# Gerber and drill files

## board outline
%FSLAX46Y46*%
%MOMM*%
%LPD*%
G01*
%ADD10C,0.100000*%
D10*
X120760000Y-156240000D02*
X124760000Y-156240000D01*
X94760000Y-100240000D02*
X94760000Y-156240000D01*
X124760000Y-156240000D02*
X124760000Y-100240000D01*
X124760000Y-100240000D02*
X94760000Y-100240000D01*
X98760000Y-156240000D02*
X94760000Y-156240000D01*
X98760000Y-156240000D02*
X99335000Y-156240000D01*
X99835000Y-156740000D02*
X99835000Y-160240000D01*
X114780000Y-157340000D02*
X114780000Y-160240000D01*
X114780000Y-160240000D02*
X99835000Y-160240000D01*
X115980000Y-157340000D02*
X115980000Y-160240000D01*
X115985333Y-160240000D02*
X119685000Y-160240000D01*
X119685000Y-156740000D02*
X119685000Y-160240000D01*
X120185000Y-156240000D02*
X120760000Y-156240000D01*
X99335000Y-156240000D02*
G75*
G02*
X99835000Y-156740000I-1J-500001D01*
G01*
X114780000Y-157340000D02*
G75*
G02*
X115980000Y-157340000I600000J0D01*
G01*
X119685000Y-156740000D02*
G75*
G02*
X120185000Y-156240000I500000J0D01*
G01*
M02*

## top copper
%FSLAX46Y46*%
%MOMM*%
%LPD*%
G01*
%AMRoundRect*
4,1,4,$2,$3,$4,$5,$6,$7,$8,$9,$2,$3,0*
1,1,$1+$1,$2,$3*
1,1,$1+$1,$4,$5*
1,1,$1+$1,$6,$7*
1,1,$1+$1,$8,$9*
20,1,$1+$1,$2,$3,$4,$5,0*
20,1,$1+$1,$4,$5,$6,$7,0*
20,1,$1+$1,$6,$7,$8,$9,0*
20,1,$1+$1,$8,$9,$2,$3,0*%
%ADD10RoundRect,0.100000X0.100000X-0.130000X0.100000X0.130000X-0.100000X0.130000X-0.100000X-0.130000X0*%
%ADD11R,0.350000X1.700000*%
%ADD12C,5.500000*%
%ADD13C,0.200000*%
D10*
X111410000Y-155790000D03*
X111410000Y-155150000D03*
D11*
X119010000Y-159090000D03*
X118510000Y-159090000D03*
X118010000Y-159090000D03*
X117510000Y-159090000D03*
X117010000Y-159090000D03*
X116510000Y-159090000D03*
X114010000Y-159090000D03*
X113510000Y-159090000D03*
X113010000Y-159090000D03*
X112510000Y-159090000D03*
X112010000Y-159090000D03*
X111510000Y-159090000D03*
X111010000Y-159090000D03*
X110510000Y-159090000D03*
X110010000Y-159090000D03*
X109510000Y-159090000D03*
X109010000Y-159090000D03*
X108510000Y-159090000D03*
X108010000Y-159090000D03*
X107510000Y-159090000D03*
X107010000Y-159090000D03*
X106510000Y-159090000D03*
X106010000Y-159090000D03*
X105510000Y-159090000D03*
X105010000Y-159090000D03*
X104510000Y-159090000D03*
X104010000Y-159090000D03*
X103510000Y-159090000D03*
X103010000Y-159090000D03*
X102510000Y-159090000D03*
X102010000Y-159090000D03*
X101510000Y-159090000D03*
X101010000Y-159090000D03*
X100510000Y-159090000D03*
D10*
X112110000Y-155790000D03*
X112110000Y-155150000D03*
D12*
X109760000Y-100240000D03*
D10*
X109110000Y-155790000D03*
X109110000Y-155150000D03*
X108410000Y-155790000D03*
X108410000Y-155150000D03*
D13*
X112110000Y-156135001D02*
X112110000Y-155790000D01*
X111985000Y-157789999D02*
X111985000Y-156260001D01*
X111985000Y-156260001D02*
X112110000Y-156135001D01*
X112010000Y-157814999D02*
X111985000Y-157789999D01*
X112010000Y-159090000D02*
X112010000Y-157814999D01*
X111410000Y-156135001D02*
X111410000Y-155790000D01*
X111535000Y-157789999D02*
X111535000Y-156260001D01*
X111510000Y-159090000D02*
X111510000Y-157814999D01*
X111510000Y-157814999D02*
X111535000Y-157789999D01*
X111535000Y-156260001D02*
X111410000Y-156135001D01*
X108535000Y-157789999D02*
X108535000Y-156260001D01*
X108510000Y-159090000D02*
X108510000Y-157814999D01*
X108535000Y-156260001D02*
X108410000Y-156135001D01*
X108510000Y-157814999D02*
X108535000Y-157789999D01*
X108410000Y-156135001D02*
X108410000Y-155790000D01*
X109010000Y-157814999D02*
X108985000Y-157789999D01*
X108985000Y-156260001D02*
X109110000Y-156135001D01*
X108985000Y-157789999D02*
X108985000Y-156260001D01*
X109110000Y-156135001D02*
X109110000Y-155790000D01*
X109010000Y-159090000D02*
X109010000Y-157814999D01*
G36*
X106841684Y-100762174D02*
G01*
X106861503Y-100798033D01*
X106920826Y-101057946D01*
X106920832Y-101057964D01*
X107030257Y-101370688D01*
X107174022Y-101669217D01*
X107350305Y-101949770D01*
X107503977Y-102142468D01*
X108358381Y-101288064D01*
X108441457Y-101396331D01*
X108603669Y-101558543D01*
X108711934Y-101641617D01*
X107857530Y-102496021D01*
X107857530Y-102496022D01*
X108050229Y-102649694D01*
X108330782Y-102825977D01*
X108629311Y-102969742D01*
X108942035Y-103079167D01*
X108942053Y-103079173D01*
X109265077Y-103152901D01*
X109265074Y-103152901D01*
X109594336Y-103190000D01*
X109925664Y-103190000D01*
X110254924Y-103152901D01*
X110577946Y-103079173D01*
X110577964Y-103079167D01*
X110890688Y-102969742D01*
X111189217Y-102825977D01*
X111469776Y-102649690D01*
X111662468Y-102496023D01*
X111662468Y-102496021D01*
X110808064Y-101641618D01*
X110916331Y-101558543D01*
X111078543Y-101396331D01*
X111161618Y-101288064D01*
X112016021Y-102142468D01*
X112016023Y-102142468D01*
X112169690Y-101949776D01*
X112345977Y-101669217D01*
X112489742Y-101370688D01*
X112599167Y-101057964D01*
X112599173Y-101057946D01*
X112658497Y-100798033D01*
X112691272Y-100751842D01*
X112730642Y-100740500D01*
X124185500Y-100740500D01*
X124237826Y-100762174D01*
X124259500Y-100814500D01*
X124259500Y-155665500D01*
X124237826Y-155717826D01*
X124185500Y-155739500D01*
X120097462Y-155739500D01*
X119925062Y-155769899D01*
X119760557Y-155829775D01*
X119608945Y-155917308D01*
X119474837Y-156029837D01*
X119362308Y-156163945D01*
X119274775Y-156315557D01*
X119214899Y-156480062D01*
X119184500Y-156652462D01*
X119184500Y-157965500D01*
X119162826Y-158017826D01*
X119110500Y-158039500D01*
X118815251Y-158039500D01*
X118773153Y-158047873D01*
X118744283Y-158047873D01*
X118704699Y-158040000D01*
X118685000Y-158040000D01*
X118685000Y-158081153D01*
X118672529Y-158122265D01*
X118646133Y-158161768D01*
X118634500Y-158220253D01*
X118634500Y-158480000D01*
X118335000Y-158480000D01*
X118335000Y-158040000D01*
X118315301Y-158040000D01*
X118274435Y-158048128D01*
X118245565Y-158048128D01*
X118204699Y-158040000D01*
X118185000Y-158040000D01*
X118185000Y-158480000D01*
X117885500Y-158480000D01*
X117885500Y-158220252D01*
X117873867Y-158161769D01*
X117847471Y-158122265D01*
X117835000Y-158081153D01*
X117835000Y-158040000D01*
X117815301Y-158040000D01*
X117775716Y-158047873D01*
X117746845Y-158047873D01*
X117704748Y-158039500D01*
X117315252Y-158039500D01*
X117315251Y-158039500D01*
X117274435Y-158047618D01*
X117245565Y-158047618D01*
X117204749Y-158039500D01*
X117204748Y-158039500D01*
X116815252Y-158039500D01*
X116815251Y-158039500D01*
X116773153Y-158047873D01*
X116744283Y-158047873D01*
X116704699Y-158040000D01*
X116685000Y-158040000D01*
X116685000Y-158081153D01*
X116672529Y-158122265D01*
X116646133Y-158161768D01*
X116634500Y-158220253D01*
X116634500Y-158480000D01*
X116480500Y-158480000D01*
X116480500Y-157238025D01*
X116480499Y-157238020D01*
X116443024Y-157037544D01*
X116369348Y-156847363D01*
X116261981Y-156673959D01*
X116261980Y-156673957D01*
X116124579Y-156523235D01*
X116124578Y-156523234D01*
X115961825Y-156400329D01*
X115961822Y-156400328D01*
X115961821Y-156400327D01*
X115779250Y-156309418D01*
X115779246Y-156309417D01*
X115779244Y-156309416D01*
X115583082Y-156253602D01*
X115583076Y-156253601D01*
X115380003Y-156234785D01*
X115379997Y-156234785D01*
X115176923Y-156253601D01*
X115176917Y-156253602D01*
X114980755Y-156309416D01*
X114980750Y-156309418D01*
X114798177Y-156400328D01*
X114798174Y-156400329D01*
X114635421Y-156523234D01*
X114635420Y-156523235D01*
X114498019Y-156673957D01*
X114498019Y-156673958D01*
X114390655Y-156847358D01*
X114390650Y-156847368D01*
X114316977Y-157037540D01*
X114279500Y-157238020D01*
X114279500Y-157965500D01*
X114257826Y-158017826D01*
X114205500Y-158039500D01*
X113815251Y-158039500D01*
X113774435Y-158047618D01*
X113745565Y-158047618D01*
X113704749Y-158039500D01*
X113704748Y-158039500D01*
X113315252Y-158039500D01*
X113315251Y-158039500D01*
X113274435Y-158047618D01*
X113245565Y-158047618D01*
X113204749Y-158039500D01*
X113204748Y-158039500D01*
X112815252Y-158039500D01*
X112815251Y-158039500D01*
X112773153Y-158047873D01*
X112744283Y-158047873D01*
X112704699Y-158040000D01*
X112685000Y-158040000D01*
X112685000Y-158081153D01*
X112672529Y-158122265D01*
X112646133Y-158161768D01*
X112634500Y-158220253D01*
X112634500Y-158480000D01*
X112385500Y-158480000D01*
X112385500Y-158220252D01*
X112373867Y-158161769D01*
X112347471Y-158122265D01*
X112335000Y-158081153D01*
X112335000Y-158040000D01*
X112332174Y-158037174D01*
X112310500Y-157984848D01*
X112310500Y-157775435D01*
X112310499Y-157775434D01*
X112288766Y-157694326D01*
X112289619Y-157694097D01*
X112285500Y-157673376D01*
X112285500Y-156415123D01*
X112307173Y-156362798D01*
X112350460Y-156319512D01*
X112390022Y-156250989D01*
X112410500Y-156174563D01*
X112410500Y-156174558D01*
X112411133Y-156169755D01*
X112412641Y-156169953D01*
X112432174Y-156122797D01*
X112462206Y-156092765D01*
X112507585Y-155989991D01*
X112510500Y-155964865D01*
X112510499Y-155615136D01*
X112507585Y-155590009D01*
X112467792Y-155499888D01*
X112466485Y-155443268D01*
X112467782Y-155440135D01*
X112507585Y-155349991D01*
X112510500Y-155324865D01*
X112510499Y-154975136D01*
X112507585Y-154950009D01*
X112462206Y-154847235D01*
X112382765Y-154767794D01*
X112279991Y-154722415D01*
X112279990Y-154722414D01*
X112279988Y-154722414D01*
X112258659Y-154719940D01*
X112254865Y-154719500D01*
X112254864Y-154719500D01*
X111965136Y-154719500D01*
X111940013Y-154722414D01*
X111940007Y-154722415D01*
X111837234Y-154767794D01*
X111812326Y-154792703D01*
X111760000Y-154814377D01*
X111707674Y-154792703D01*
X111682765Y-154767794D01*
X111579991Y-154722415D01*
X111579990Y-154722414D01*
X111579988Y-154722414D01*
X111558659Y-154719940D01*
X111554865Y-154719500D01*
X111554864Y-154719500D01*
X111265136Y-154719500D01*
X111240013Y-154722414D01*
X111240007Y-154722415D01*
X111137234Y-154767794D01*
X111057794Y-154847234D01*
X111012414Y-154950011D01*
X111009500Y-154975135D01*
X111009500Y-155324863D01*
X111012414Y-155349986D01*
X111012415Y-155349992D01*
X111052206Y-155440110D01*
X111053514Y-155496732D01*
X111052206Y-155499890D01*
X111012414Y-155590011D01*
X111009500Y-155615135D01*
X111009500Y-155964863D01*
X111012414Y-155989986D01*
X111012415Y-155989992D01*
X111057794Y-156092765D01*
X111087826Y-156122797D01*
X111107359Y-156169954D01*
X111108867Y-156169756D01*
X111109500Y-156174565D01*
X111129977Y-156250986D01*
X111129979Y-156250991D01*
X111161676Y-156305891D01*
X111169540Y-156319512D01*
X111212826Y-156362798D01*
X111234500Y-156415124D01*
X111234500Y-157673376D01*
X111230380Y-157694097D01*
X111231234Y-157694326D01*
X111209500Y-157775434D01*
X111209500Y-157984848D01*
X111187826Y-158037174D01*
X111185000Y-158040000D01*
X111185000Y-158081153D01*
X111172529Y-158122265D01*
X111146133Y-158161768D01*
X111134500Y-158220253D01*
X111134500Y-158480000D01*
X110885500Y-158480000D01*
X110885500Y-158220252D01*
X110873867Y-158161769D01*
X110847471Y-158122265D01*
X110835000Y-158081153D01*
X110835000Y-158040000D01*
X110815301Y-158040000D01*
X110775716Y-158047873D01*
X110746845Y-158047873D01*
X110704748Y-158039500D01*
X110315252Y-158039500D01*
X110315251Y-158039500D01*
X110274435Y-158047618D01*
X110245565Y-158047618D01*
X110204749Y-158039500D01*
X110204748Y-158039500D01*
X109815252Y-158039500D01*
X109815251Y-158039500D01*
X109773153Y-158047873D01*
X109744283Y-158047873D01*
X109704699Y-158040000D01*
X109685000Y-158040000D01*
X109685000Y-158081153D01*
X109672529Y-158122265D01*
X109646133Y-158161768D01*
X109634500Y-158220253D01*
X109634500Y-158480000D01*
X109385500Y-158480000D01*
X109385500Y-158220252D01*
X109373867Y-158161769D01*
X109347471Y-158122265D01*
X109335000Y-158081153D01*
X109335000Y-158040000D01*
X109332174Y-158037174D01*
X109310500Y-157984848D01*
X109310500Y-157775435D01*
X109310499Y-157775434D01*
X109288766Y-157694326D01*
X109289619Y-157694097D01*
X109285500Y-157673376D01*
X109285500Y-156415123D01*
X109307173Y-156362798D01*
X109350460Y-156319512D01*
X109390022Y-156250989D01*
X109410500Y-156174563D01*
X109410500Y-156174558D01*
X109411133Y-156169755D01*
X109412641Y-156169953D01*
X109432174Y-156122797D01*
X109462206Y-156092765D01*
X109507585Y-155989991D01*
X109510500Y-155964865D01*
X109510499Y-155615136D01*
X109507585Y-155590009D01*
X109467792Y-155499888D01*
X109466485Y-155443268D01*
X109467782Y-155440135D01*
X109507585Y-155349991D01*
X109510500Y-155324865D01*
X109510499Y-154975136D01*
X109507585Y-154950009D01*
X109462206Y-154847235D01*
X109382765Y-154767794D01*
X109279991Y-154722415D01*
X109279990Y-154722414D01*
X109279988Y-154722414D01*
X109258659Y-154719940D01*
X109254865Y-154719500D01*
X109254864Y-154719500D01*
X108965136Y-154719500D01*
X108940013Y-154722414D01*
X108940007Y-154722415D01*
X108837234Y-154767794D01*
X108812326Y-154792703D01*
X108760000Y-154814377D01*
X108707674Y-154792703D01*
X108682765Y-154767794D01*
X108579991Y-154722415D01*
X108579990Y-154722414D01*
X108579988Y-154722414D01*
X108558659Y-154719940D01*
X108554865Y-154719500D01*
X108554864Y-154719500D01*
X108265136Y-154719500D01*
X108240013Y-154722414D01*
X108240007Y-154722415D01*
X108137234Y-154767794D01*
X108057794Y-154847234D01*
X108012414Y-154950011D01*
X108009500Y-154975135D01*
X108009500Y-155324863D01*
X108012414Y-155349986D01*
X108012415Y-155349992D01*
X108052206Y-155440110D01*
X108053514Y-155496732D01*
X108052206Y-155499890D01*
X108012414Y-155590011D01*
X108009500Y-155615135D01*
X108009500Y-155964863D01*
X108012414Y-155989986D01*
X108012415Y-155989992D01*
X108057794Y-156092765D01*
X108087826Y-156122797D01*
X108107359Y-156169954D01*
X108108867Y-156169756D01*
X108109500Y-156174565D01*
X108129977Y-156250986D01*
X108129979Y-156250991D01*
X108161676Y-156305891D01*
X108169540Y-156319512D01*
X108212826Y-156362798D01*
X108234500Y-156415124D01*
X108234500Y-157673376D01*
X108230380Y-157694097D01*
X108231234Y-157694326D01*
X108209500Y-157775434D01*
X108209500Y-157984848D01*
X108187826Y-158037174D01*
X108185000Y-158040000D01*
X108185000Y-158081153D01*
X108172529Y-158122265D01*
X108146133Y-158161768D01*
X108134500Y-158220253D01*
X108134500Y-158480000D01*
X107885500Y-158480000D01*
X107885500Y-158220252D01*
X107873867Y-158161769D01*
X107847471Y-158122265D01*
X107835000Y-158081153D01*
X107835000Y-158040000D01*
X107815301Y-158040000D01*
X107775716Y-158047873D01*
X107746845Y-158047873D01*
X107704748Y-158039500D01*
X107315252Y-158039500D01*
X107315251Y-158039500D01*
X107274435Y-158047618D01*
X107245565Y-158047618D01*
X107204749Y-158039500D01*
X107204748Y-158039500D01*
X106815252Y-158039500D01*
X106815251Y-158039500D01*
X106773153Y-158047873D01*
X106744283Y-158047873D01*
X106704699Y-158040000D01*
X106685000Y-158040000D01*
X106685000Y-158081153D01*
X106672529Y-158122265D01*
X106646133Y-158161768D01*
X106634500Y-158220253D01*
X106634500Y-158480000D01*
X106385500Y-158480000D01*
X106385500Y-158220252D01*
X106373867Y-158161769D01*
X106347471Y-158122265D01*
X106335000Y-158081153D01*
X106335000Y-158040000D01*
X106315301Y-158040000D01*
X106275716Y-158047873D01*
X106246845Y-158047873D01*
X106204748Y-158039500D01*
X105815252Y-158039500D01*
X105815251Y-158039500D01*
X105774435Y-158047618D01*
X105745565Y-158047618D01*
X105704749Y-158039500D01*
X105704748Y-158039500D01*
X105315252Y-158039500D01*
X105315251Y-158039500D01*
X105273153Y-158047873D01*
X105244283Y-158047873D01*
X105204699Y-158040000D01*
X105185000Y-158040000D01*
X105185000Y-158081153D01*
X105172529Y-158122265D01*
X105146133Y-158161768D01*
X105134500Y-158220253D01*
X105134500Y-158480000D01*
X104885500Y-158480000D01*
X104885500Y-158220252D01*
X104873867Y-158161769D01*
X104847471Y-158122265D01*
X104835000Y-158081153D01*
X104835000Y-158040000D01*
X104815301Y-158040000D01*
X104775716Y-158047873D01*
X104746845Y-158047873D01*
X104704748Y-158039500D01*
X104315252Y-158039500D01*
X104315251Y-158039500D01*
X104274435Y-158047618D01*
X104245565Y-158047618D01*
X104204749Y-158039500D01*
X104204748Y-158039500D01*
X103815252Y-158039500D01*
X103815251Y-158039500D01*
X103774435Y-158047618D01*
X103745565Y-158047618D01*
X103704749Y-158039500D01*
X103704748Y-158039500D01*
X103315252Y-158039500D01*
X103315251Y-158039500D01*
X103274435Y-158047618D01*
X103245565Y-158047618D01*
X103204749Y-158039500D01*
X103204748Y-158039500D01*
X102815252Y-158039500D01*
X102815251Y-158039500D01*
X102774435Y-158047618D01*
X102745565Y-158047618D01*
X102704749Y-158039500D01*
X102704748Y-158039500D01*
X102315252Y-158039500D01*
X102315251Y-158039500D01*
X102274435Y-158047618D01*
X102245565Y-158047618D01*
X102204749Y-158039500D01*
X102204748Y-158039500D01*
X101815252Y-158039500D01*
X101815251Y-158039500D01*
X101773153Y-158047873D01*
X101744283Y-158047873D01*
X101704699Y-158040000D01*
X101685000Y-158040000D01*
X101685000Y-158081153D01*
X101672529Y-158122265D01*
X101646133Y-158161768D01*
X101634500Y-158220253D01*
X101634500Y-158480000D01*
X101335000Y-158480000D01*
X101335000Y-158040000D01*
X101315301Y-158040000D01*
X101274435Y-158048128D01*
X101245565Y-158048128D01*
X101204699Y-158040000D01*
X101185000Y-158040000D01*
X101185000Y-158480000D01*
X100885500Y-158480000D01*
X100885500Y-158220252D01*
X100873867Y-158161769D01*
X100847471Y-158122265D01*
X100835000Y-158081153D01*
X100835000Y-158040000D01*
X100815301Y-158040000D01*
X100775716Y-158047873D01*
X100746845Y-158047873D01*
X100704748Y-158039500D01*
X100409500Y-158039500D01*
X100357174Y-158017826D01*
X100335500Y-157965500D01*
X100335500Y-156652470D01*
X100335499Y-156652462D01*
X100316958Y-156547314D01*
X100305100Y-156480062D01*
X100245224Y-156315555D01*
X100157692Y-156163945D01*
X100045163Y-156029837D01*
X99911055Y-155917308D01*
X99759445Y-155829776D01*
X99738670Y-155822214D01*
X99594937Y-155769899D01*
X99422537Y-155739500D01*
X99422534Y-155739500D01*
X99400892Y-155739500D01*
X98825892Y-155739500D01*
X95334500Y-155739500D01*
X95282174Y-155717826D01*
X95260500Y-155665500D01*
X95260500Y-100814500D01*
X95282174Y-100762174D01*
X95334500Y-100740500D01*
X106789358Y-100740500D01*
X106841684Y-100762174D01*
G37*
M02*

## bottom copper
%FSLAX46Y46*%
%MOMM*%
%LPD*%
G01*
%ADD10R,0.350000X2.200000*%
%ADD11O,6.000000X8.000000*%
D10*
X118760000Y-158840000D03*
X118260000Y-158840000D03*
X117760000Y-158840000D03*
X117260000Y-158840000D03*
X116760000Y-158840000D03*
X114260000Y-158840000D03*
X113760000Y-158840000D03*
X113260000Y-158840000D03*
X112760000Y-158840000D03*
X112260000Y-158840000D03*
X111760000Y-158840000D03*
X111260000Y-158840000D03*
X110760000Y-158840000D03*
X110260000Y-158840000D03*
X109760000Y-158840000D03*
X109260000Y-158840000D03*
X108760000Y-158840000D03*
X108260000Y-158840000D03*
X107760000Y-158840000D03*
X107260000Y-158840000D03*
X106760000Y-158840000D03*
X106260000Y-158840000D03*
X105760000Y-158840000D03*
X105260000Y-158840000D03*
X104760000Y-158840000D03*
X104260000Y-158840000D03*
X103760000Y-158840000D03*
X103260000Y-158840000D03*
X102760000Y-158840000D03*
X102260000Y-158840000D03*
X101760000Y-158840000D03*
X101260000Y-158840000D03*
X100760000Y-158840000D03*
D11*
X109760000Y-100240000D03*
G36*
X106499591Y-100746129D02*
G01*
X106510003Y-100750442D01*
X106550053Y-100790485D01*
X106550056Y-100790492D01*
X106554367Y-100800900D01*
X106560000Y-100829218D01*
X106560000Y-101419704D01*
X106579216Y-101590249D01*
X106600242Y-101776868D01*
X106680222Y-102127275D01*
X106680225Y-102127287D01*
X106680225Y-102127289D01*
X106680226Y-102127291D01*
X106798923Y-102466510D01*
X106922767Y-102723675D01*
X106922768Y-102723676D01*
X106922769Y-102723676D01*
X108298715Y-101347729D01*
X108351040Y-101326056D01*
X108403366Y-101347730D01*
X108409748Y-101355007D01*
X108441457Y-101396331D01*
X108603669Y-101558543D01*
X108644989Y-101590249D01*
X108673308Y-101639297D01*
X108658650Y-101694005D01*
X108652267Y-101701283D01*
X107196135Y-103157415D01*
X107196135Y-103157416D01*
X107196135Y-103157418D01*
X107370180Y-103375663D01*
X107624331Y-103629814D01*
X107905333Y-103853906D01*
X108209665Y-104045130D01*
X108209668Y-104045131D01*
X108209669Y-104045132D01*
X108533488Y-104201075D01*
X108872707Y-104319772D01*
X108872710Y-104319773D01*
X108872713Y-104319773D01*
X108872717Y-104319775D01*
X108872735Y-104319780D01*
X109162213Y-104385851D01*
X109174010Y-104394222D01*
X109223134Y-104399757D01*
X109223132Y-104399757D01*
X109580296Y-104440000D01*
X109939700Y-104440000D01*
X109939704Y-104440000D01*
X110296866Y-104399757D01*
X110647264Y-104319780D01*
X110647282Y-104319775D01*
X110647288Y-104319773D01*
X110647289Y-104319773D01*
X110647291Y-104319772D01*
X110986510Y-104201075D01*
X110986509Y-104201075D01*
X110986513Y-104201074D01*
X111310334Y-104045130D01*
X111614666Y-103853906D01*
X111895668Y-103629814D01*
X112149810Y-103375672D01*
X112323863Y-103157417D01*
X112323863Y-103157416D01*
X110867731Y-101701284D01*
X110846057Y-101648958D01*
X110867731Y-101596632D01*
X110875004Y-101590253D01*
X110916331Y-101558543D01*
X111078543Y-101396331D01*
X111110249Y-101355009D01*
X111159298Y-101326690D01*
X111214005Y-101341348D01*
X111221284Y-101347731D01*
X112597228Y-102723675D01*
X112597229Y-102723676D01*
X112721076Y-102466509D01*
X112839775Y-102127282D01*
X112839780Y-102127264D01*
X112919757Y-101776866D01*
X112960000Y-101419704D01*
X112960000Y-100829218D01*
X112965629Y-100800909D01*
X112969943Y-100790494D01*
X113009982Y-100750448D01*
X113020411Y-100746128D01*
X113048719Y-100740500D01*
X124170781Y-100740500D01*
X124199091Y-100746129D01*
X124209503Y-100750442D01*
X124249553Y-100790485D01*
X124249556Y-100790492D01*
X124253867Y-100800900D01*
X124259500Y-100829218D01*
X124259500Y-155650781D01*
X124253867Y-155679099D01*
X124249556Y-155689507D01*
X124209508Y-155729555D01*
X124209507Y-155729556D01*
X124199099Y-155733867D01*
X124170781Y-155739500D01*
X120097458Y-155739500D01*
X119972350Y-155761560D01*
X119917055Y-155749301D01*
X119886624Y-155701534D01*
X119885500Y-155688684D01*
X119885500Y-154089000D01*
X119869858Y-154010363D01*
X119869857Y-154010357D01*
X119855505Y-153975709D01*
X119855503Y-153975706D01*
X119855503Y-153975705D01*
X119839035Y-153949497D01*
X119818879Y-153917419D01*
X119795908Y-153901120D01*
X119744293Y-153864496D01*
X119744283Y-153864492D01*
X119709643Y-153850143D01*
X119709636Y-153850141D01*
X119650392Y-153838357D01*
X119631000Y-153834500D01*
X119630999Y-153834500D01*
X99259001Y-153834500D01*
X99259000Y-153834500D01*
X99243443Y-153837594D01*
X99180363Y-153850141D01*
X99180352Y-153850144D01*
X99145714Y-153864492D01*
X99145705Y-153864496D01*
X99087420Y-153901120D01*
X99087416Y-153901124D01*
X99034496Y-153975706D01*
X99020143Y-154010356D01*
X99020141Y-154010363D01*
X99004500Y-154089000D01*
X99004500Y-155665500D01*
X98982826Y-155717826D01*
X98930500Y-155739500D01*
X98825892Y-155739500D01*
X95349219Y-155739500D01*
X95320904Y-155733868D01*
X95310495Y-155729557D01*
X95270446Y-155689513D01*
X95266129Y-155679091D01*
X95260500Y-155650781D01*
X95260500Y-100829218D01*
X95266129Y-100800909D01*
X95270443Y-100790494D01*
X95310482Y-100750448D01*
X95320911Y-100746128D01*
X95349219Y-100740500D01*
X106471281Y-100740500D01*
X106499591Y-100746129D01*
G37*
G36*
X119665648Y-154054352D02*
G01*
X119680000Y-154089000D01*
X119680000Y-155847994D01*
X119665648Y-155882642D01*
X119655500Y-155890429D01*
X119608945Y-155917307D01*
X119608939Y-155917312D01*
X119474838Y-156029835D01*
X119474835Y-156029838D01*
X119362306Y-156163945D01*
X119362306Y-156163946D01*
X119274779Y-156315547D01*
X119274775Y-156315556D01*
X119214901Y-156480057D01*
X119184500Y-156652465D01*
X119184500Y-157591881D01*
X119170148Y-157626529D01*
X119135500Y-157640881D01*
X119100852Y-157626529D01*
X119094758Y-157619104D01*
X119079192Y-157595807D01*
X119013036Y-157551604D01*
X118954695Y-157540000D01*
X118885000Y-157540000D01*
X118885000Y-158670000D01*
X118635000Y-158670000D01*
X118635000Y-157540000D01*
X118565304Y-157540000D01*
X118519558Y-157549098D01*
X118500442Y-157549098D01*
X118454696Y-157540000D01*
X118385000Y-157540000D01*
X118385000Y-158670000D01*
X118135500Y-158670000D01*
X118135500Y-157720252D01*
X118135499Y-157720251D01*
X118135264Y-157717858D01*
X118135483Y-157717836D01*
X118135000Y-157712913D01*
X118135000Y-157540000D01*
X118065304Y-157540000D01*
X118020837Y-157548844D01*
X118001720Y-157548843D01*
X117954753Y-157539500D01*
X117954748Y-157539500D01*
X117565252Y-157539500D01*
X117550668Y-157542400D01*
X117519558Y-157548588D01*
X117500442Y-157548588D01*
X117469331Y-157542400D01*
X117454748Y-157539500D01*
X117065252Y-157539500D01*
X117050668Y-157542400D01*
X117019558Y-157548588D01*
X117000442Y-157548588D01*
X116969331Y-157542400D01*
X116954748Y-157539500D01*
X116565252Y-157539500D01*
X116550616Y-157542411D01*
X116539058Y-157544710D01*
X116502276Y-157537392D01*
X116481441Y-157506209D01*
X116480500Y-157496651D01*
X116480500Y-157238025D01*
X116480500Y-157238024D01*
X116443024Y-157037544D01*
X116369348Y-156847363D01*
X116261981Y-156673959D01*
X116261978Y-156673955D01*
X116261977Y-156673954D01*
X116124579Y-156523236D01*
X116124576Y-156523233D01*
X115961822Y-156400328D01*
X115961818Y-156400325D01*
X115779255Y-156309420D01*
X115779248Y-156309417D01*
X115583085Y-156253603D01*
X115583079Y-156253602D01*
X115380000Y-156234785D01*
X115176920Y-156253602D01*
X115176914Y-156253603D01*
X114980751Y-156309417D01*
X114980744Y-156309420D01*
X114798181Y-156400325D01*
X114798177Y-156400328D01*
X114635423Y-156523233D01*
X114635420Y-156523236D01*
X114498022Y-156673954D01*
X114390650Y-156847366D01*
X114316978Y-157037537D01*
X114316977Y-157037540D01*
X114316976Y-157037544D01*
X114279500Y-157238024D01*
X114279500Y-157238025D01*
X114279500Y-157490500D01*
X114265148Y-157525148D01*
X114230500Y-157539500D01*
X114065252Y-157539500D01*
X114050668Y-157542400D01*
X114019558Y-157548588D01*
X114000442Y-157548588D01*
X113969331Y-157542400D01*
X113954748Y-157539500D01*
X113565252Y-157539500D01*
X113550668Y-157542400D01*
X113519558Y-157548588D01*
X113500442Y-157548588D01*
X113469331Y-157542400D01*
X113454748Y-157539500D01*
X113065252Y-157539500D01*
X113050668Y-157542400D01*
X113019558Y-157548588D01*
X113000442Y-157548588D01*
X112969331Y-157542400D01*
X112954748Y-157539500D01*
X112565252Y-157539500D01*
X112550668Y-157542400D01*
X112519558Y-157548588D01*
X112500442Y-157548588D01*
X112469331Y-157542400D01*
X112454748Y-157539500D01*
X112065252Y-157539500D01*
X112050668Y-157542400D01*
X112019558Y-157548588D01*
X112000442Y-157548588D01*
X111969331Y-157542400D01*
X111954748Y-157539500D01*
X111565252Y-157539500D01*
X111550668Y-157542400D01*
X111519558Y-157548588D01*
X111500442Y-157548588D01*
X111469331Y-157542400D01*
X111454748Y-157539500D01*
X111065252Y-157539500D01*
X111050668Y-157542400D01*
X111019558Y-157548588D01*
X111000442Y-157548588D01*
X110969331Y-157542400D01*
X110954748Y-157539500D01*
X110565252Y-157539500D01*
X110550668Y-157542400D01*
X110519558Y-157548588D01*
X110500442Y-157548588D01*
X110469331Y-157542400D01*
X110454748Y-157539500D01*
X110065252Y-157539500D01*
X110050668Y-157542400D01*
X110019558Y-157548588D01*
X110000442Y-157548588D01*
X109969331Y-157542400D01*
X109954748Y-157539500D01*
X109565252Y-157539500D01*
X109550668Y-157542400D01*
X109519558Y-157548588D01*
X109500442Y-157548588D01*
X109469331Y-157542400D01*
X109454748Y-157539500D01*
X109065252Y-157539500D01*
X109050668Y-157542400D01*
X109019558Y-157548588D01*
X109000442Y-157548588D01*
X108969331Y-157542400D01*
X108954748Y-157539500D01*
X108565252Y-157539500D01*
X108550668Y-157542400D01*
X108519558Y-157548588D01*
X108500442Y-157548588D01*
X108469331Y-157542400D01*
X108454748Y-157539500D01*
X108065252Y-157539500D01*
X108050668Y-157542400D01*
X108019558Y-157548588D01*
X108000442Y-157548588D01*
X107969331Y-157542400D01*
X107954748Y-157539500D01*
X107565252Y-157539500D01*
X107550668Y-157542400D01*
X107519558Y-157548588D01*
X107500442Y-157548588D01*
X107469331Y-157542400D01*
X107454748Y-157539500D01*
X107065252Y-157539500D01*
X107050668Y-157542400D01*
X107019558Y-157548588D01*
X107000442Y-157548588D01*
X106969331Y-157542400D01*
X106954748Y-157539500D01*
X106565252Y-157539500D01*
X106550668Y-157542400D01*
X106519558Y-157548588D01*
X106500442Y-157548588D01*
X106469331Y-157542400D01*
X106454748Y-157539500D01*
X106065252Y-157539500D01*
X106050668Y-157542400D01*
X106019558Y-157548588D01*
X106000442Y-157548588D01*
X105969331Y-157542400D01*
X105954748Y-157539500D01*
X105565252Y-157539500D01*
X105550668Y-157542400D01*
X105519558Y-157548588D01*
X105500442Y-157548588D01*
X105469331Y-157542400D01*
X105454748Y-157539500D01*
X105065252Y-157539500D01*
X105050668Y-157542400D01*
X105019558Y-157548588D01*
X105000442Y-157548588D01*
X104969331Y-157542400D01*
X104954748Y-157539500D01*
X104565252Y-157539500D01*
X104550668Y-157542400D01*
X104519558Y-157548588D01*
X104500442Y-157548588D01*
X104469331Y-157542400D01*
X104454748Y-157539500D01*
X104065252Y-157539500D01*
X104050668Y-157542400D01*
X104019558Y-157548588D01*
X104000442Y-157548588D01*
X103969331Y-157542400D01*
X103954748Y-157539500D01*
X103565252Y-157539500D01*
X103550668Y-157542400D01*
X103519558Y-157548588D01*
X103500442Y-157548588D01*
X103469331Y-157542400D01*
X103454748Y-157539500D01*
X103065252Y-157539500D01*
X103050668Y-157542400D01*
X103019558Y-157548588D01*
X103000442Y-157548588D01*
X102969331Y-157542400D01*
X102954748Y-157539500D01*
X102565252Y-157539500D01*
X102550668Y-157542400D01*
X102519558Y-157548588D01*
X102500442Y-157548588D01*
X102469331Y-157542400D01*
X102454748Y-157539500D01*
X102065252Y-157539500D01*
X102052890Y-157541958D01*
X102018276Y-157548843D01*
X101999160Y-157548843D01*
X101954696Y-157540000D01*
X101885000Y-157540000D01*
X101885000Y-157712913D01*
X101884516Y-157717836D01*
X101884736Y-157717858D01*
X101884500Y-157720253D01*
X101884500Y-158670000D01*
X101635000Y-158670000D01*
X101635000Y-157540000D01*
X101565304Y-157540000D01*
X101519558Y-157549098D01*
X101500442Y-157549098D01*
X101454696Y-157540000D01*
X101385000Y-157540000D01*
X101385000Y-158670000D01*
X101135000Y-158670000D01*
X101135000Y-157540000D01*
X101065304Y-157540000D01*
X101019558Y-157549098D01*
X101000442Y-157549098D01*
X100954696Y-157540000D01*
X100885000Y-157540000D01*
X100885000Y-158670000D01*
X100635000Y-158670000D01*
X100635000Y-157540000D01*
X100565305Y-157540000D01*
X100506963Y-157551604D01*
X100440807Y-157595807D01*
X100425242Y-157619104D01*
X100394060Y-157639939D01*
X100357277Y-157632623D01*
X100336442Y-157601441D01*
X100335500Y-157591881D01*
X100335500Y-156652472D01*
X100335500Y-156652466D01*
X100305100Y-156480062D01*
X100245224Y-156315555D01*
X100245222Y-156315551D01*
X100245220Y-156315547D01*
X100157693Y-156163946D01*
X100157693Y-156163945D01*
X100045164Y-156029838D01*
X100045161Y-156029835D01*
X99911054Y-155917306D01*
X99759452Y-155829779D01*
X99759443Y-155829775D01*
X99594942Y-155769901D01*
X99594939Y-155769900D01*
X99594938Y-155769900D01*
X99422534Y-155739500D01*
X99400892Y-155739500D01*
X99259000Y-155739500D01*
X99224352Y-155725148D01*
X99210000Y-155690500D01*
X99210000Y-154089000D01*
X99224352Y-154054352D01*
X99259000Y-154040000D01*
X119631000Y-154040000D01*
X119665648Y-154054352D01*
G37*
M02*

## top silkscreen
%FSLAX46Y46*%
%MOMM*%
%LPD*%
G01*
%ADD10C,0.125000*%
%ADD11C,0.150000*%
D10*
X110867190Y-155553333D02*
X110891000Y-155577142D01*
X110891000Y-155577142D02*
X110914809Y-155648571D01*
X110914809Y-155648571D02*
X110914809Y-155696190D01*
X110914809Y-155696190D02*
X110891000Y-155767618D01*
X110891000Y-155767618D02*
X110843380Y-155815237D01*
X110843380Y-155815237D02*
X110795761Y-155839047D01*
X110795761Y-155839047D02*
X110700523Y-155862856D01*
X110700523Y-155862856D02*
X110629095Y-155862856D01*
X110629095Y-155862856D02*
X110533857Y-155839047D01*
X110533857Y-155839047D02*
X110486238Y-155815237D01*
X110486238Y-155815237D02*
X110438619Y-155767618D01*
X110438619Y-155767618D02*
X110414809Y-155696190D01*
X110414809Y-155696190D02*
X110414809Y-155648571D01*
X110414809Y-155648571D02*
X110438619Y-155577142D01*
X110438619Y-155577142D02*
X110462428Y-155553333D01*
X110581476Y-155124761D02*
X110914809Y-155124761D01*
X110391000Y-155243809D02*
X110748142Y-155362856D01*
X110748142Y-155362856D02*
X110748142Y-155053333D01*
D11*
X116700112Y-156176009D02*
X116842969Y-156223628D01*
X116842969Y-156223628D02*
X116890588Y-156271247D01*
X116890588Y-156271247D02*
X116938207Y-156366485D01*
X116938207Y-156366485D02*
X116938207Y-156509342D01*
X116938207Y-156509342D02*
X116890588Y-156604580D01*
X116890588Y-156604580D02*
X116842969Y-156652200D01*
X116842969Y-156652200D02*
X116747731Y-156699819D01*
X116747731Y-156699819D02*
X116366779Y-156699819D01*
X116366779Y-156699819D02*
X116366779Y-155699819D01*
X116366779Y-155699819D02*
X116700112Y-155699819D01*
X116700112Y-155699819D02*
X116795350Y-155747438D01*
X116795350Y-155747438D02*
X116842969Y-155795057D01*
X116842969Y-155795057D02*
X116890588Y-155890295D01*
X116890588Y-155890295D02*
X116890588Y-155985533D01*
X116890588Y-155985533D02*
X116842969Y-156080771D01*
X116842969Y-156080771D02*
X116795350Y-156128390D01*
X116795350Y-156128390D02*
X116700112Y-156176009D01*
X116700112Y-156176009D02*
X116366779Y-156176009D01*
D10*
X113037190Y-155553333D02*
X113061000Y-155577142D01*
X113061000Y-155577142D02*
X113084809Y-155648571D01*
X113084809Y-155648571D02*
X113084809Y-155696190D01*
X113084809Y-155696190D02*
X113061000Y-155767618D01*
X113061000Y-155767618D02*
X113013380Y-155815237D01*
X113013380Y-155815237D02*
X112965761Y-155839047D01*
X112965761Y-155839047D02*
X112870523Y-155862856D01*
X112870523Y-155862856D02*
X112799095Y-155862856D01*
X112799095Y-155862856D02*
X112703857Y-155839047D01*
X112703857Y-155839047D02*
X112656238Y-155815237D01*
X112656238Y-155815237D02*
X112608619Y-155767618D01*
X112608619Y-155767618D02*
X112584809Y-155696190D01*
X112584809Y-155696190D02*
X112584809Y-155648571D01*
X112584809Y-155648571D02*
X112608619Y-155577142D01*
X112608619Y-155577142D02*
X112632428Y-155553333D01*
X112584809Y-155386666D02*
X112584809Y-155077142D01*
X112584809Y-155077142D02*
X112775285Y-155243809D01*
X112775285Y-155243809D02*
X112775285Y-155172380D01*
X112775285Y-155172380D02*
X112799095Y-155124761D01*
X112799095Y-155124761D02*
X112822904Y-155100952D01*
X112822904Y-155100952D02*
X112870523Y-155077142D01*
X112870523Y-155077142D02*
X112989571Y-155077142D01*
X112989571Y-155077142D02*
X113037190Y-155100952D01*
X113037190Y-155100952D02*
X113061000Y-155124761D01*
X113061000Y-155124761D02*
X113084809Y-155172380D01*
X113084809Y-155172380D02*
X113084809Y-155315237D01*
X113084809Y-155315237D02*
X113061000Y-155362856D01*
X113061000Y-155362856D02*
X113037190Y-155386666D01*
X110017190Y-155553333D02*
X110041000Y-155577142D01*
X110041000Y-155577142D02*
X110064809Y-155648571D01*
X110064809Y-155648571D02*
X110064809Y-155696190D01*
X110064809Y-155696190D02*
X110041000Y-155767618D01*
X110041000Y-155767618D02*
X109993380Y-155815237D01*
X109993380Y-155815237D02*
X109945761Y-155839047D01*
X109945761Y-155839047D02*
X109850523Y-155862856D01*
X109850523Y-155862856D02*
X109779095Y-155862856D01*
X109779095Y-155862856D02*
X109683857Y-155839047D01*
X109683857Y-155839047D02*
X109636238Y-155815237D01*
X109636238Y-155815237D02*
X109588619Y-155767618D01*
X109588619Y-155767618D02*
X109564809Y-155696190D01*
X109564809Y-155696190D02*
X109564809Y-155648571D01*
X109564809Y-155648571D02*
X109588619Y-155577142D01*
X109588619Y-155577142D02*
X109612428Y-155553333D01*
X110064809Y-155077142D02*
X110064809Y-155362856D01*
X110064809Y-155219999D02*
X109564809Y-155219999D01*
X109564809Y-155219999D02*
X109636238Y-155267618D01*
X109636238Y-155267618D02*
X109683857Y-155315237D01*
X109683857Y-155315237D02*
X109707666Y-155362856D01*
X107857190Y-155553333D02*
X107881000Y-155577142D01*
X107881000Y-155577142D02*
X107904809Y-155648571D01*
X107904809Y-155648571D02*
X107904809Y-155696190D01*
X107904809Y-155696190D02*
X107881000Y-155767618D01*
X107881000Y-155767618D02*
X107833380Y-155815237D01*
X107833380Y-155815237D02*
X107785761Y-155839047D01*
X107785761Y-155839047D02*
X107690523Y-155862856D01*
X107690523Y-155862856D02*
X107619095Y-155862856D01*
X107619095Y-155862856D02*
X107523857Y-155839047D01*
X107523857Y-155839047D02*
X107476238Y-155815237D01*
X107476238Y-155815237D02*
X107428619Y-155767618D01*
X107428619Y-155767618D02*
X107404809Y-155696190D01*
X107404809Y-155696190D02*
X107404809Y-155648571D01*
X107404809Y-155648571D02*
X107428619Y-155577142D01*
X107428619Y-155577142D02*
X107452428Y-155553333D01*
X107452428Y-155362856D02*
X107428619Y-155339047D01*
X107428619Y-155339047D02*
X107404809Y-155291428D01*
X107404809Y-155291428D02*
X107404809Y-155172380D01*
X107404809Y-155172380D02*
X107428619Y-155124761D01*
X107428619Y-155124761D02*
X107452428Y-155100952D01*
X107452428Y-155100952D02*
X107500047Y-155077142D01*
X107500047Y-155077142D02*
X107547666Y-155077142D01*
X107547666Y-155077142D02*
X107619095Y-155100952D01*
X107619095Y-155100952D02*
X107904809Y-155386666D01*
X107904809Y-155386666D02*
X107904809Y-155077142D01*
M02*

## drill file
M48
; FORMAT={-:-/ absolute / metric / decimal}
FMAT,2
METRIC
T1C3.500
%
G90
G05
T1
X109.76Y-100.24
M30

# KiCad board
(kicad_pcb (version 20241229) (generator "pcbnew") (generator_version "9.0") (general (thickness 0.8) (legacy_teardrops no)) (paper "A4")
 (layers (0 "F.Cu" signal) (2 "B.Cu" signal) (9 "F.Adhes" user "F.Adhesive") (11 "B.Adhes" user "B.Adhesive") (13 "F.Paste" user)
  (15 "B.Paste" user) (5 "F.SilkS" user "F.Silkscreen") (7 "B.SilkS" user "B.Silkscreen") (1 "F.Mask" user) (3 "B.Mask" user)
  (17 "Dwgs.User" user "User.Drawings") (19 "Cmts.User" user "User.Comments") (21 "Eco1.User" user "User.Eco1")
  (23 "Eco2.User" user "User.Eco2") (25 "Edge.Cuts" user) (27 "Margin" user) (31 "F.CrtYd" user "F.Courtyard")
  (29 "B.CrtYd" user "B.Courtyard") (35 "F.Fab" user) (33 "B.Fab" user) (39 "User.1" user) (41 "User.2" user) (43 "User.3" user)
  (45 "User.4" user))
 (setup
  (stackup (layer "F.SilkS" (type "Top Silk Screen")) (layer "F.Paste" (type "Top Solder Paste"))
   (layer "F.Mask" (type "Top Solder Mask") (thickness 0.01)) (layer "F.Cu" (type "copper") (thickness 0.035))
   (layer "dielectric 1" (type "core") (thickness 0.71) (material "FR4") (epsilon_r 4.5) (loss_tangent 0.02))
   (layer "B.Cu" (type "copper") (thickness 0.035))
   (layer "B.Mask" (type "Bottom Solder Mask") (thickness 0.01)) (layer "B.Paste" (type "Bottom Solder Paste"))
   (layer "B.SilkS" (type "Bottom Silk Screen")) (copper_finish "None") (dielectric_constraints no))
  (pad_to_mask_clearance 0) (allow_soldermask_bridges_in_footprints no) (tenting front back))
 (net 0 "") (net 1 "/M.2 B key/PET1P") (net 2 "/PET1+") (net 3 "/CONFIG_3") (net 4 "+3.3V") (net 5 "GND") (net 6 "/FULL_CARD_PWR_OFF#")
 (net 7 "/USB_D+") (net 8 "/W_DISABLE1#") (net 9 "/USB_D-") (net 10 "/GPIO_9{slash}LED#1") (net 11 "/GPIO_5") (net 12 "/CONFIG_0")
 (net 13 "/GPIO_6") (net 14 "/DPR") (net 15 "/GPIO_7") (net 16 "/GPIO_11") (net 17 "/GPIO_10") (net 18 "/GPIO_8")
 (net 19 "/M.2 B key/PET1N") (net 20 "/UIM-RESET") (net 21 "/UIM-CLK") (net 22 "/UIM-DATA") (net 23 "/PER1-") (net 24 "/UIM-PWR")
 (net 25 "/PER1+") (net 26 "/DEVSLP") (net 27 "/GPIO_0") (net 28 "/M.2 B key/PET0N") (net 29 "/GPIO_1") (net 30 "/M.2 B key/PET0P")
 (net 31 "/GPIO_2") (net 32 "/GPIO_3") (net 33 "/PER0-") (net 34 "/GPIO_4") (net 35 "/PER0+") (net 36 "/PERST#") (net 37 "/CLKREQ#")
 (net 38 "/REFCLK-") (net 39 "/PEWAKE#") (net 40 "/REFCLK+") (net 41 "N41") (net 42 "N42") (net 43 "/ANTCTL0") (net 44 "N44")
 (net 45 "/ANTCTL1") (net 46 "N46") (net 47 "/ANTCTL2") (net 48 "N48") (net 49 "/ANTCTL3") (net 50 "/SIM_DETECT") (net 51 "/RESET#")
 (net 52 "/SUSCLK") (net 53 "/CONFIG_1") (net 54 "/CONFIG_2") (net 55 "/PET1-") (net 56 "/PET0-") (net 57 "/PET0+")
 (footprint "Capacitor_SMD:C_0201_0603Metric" (layer "F.Cu") (at 111.41 155.47 90)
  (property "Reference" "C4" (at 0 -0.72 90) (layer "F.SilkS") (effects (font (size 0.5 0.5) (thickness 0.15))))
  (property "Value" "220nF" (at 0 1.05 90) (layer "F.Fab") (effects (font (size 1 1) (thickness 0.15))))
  (pad "" smd roundrect (at -0.345 0 90) (size 0.318 0.36) (layers "F.Paste") (roundrect_rratio 0.25))
  (pad "" smd roundrect (at 0.345 0 90) (size 0.318 0.36) (layers "F.Paste") (roundrect_rratio 0.25))
  (pad "1" smd roundrect (at -0.32 0 90) (size 0.46 0.4) (layers "F.Cu" "F.Mask") (roundrect_rratio 0.25) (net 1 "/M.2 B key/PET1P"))
  (pad "2" smd roundrect (at 0.32 0 90) (size 0.46 0.4) (layers "F.Cu" "F.Mask") (roundrect_rratio 0.25) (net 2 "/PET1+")))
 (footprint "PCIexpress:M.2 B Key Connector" (layer "F.Cu") (at 109.76 159.13)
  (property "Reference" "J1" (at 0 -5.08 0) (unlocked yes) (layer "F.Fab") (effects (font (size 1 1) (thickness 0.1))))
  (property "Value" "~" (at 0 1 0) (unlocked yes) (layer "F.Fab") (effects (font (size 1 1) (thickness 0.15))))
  (fp_line (start -11 -2.89) (end -10.425 -2.89) (stroke (width 0.1) (type default)) (layer "Edge.Cuts"))
  (fp_line (start -9.925 -2.39) (end -9.925 1.11) (stroke (width 0.1) (type default)) (layer "Edge.Cuts"))
  (fp_line (start 5.02 -1.79) (end 5.02 1.11) (stroke (width 0.1) (type default)) (layer "Edge.Cuts"))
  (fp_line (start 5.02 1.11) (end -9.925 1.11) (stroke (width 0.1) (type default)) (layer "Edge.Cuts"))
  (fp_line (start 6.22 -1.79) (end 6.22 1.11) (stroke (width 0.1) (type default)) (layer "Edge.Cuts"))
  (fp_line (start 6.225333 1.11) (end 9.925 1.11) (stroke (width 0.1) (type default)) (layer "Edge.Cuts"))
  (fp_line (start 9.925 -2.39) (end 9.925 1.11) (stroke (width 0.1) (type default)) (layer "Edge.Cuts"))
  (fp_line (start 10.425 -2.89) (end 11 -2.89) (stroke (width 0.1) (type default)) (layer "Edge.Cuts"))
  (fp_arc (start -10.425 -2.89) (mid -10.071447 -2.743553) (end -9.925 -2.39) (stroke (width 0.1) (type default)) (layer "Edge.Cuts"))
  (fp_arc (start 5.02 -1.79) (mid 5.62 -2.39) (end 6.22 -1.79) (stroke (width 0.1) (type default)) (layer "Edge.Cuts"))
  (fp_arc (start 9.925 -2.39) (mid 10.071447 -2.743553) (end 10.425 -2.89) (stroke (width 0.1) (type default)) (layer "Edge.Cuts"))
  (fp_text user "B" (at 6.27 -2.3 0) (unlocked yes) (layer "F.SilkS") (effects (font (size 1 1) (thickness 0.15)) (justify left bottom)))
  (pad "1" smd rect (at 9.25 -0.04 180) (size 0.35 1.7) (layers "F.Cu") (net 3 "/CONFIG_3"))
  (pad "2" smd rect (at 9 -0.29 180) (size 0.35 2.2) (layers "B.Cu") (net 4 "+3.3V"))
  (pad "3" smd rect (at 8.75 -0.04 180) (size 0.35 1.7) (layers "F.Cu") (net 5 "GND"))
  (pad "4" smd rect (at 8.5 -0.29 180) (size 0.35 2.2) (layers "B.Cu") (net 4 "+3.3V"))
  (pad "5" smd rect (at 8.25 -0.04 180) (size 0.35 1.7) (layers "F.Cu") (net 5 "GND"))
  (pad "6" smd rect (at 8 -0.29 180) (size 0.35 2.2) (layers "B.Cu") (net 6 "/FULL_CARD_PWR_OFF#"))
  (pad "7" smd rect (at 7.75 -0.04 180) (size 0.35 1.7) (layers "F.Cu") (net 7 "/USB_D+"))
  (pad "8" smd rect (at 7.5 -0.29 180) (size 0.35 2.2) (layers "B.Cu") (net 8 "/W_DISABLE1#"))
  (pad "9" smd rect (at 7.25 -0.04 180) (size 0.35 1.7) (layers "F.Cu") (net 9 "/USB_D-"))
  (pad "10" smd rect (at 7 -0.29 180) (size 0.35 2.2) (layers "B.Cu") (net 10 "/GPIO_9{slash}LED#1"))
  (pad "11" smd rect (at 6.75 -0.04 180) (size 0.35 1.7) (layers "F.Cu") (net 5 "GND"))
  (pad "20" smd rect (at 4.5 -0.29 180) (size 0.35 2.2) (layers "B.Cu") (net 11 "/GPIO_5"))
  (pad "21" smd rect (at 4.25 -0.04 180) (size 0.35 1.7) (layers "F.Cu") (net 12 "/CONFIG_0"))
  (pad "22" smd rect (at 4 -0.29 180) (size 0.35 2.2) (layers "B.Cu") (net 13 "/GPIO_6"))
  (pad "23" smd rect (at 3.75 -0.04 180) (size 0.35 1.7) (layers "F.Cu") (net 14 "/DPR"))
  (pad "24" smd rect (at 3.5 -0.29 180) (size 0.35 2.2) (layers "B.Cu") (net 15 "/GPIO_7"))
  (pad "25" smd rect (at 3.25 -0.04 180) (size 0.35 1.7) (layers "F.Cu") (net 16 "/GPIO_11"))
  (pad "26" smd rect (at 3 -0.29 180) (size 0.35 2.2) (layers "B.Cu") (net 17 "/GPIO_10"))
  (pad "27" smd rect (at 2.75 -0.04 180) (size 0.35 1.7) (layers "F.Cu") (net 5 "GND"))
  (pad "28" smd rect (at 2.5 -0.29 180) (size 0.35 2.2) (layers "B.Cu") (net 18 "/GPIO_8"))
  (pad "29" smd rect (at 2.25 -0.04 180) (size 0.35 1.7) (layers "F.Cu") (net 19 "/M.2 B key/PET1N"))
  (pad "30" smd rect (at 2 -0.29 180) (size 0.35 2.2) (layers "B.Cu") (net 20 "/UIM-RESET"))
  (pad "31" smd rect (at 1.75 -0.04 180) (size 0.35 1.7) (layers "F.Cu") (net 1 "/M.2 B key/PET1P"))
  (pad "32" smd rect (at 1.5 -0.29 180) (size 0.35 2.2) (layers "B.Cu") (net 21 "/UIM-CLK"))
  (pad "33" smd rect (at 1.25 -0.04 180) (size 0.35 1.7) (layers "F.Cu") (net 5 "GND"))
  (pad "34" smd rect (at 1 -0.29 180) (size 0.35 2.2) (layers "B.Cu") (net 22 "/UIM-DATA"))
  (pad "35" smd rect (at 0.75 -0.04 180) (size 0.35 1.7) (layers "F.Cu") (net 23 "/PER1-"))
  (pad "36" smd rect (at 0.5 -0.29 180) (size 0.35 2.2) (layers "B.Cu") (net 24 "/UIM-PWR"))
  (pad "37" smd rect (at 0.25 -0.04 180) (size 0.35 1.7) (layers "F.Cu") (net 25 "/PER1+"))
  (pad "38" smd rect (at 0 -0.29 180) (size 0.35 2.2) (layers "B.Cu") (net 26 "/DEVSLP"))
  (pad "39" smd rect (at -0.25 -0.04 180) (size 0.35 1.7) (layers "F.Cu") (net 5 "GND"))
  (pad "40" smd rect (at -0.5 -0.29 180) (size 0.35 2.2) (layers "B.Cu") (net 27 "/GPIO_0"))
  (pad "41" smd rect (at -0.75 -0.04 180) (size 0.35 1.7) (layers "F.Cu") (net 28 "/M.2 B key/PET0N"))
  (pad "42" smd rect (at -1 -0.29 180) (size 0.35 2.2) (layers "B.Cu") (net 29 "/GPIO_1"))
  (pad "43" smd rect (at -1.25 -0.04 180) (size 0.35 1.7) (layers "F.Cu") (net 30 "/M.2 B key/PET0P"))
  (pad "44" smd rect (at -1.5 -0.29 180) (size 0.35 2.2) (layers "B.Cu") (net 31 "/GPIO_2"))
  (pad "45" smd rect (at -1.75 -0.04 180) (size 0.35 1.7) (layers "F.Cu") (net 5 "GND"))
  (pad "46" smd rect (at -2 -0.29 180) (size 0.35 2.2) (layers "B.Cu") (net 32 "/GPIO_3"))
  (pad "47" smd rect (at -2.25 -0.04 180) (size 0.35 1.7) (layers "F.Cu") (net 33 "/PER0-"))
  (pad "48" smd rect (at -2.5 -0.29 180) (size 0.35 2.2) (layers "B.Cu") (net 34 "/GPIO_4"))
  (pad "49" smd rect (at -2.75 -0.04 180) (size 0.35 1.7) (layers "F.Cu") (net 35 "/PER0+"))
  (pad "50" smd rect (at -3 -0.29 180) (size 0.35 2.2) (layers "B.Cu") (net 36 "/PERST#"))
  (pad "51" smd rect (at -3.25 -0.04 180) (size 0.35 1.7) (layers "F.Cu") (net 5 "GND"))
  (pad "52" smd rect (at -3.5 -0.29 180) (size 0.35 2.2) (layers "B.Cu") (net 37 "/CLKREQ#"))
  (pad "53" smd rect (at -3.75 -0.04 180) (size 0.35 1.7) (layers "F.Cu") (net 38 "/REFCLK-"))
  (pad "54" smd rect (at -4 -0.29 180) (size 0.35 2.2) (layers "B.Cu") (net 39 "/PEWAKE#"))
  (pad "55" smd rect (at -4.25 -0.04 180) (size 0.35 1.7) (layers "F.Cu") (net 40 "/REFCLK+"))
  (pad "56" smd rect (at -4.5 -0.29 180) (size 0.35 2.2) (layers "B.Cu") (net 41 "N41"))
  (pad "57" smd rect (at -4.75 -0.04 180) (size 0.35 1.7) (layers "F.Cu") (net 5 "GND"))
  (pad "58" smd rect (at -5 -0.29 180) (size 0.35 2.2) (layers "B.Cu") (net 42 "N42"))
  (pad "59" smd rect (at -5.25 -0.04 180) (size 0.35 1.7) (layers "F.Cu") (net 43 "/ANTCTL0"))
  (pad "60" smd rect (at -5.5 -0.29 180) (size 0.35 2.2) (layers "B.Cu") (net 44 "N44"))
  (pad "61" smd rect (at -5.75 -0.04 180) (size 0.35 1.7) (layers "F.Cu") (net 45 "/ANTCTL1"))
  (pad "62" smd rect (at -6 -0.29 180) (size 0.35 2.2) (layers "B.Cu") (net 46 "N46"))
  (pad "63" smd rect (at -6.25 -0.04 180) (size 0.35 1.7) (layers "F.Cu") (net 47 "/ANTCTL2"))
  (pad "64" smd rect (at -6.5 -0.29 180) (size 0.35 2.2) (layers "B.Cu") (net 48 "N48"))
  (pad "65" smd rect (at -6.75 -0.04 180) (size 0.35 1.7) (layers "F.Cu") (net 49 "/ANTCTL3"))
  (pad "66" smd rect (at -7 -0.29 180) (size 0.35 2.2) (layers "B.Cu") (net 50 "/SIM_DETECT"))
  (pad "67" smd rect (at -7.25 -0.04 180) (size 0.35 1.7) (layers "F.Cu") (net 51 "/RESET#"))
  (pad "68" smd rect (at -7.5 -0.29 180) (size 0.35 2.2) (layers "B.Cu") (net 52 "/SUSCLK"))
  (pad "69" smd rect (at -7.75 -0.04 180) (size 0.35 1.7) (layers "F.Cu") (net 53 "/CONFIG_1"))
  (pad "70" smd rect (at -8 -0.29 180) (size 0.35 2.2) (layers "B.Cu") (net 4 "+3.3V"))
  (pad "71" smd rect (at -8.25 -0.04 180) (size 0.35 1.7) (layers "F.Cu") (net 5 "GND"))
  (pad "72" smd rect (at -8.5 -0.29 180) (size 0.35 2.2) (layers "B.Cu") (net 4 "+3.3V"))
  (pad "73" smd rect (at -8.75 -0.04 180) (size 0.35 1.7) (layers "F.Cu") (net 5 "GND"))
  (pad "74" smd rect (at -9 -0.29 180) (size 0.35 2.2) (layers "B.Cu") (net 4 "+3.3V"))
  (pad "75" smd rect (at -9.25 -0.04 180) (size 0.35 1.7) (layers "F.Cu") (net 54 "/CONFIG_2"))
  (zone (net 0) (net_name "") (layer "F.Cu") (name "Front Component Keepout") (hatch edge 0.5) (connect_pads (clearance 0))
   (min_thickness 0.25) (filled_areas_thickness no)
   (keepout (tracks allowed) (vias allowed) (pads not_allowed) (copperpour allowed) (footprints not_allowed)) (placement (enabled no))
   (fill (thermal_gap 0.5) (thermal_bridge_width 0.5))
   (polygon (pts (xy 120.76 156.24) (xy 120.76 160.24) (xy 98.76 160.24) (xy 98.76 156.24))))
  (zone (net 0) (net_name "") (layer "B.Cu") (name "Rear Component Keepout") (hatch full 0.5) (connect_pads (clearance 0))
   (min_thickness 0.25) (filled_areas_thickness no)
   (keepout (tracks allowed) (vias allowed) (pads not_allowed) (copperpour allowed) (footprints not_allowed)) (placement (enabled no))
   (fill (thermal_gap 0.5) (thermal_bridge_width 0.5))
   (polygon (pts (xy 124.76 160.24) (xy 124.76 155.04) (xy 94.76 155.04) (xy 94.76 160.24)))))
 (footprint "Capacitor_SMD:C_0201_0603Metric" (layer "F.Cu") (at 112.11 155.47 90)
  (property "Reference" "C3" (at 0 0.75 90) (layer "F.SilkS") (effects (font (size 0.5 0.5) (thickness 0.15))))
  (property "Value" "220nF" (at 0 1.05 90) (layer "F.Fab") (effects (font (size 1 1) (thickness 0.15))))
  (pad "" smd roundrect (at -0.345 0 90) (size 0.318 0.36) (layers "F.Paste") (roundrect_rratio 0.25))
  (pad "" smd roundrect (at 0.345 0 90) (size 0.318 0.36) (layers "F.Paste") (roundrect_rratio 0.25))
  (pad "1" smd roundrect (at -0.32 0 90) (size 0.46 0.4) (layers "F.Cu" "F.Mask") (roundrect_rratio 0.25) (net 19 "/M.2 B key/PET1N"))
  (pad "2" smd roundrect (at 0.32 0 90) (size 0.46 0.4) (layers "F.Cu" "F.Mask") (roundrect_rratio 0.25) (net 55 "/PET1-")))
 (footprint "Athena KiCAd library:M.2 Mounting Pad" (layer "F.Cu") (at 109.76 100.24)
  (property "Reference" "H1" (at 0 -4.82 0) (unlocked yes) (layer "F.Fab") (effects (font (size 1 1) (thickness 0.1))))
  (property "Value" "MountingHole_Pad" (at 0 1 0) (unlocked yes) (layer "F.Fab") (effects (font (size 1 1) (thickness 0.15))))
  (pad "1" thru_hole circle (at 0 0) (size 5.5 5.5) (drill 3.5) (layers "*.Cu" "*.Mask") (remove_unused_layers no) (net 5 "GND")
   (padstack (mode front_inner_back)
    (layer "Inner" (shape circle) (size 5.5 5.5) (zone_connect -1))
    (layer "B.Cu" (shape oval) (size 6 8) (thermal_bridge_angle 45) (zone_connect -1)))))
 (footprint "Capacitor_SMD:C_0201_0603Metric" (layer "F.Cu") (at 109.11 155.47 90)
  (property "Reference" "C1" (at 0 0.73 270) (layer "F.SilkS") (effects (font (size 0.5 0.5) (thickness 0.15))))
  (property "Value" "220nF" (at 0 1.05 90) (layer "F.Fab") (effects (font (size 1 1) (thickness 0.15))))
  (pad "" smd roundrect (at -0.345 0 90) (size 0.318 0.36) (layers "F.Paste") (roundrect_rratio 0.25))
  (pad "" smd roundrect (at 0.345 0 90) (size 0.318 0.36) (layers "F.Paste") (roundrect_rratio 0.25))
  (pad "1" smd roundrect (at -0.32 0 90) (size 0.46 0.4) (layers "F.Cu" "F.Mask") (roundrect_rratio 0.25) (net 28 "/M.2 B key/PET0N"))
  (pad "2" smd roundrect (at 0.32 0 90) (size 0.46 0.4) (layers "F.Cu" "F.Mask") (roundrect_rratio 0.25) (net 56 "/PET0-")))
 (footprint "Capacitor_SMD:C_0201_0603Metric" (layer "F.Cu") (at 108.41 155.47 90)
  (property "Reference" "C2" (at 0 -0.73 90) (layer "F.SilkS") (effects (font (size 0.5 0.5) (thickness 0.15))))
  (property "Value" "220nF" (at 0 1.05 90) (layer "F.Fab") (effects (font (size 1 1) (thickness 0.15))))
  (pad "" smd roundrect (at -0.345 0 90) (size 0.318 0.36) (layers "F.Paste") (roundrect_rratio 0.25))
  (pad "" smd roundrect (at 0.345 0 90) (size 0.318 0.36) (layers "F.Paste") (roundrect_rratio 0.25))
  (pad "1" smd roundrect (at -0.32 0 90) (size 0.46 0.4) (layers "F.Cu" "F.Mask") (roundrect_rratio 0.25) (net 30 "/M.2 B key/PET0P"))
  (pad "2" smd roundrect (at 0.32 0 90) (size 0.46 0.4) (layers "F.Cu" "F.Mask") (roundrect_rratio 0.25) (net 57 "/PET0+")))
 (gr_line (start 120.76 156.24) (end 124.76 156.24) (stroke (width 0.1) (type default)) (layer "Edge.Cuts"))
 (gr_line (start 94.76 100.24) (end 94.76 156.24) (stroke (width 0.1) (type default)) (layer "Edge.Cuts"))
 (gr_line (start 124.76 156.24) (end 124.76 100.24) (stroke (width 0.1) (type default)) (layer "Edge.Cuts"))
 (gr_line (start 124.76 100.24) (end 94.76 100.24) (stroke (width 0.1) (type default)) (layer "Edge.Cuts"))
 (gr_line (start 98.76 156.24) (end 94.76 156.24) (stroke (width 0.1) (type default)) (layer "Edge.Cuts"))
 (segment (start 112.11 156.135001) (end 112.11 155.79) (width 0.2) (layer "F.Cu") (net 19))
 (segment (start 111.985 157.789999) (end 111.985 156.260001) (width 0.2) (layer "F.Cu") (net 19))
 (segment (start 111.985 156.260001) (end 112.11 156.135001) (width 0.2) (layer "F.Cu") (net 19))
 (segment (start 112.01 157.814999) (end 111.985 157.789999) (width 0.2) (layer "F.Cu") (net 19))
 (segment (start 112.01 159.09) (end 112.01 157.814999) (width 0.2) (layer "F.Cu") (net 19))
 (segment (start 111.41 156.135001) (end 111.41 155.79) (width 0.2) (layer "F.Cu") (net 1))
 (segment (start 111.535 157.789999) (end 111.535 156.260001) (width 0.2) (layer "F.Cu") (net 1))
 (segment (start 111.51 159.09) (end 111.51 157.814999) (width 0.2) (layer "F.Cu") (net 1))
 (segment (start 111.51 157.814999) (end 111.535 157.789999) (width 0.2) (layer "F.Cu") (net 1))
 (segment (start 111.535 156.260001) (end 111.41 156.135001) (width 0.2) (layer "F.Cu") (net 1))
 (segment (start 108.535 157.789999) (end 108.535 156.260001) (width 0.2) (layer "F.Cu") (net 30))
 (segment (start 108.51 159.09) (end 108.51 157.814999) (width 0.2) (layer "F.Cu") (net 30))
 (segment (start 108.535 156.260001) (end 108.41 156.135001) (width 0.2) (layer "F.Cu") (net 30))
 (segment (start 108.51 157.814999) (end 108.535 157.789999) (width 0.2) (layer "F.Cu") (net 30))
 (segment (start 108.41 156.135001) (end 108.41 155.79) (width 0.2) (layer "F.Cu") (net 30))
 (segment (start 109.01 157.814999) (end 108.985 157.789999) (width 0.2) (layer "F.Cu") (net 28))
 (segment (start 108.985 156.260001) (end 109.11 156.135001) (width 0.2) (layer "F.Cu") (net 28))
 (segment (start 108.985 157.789999) (end 108.985 156.260001) (width 0.2) (layer "F.Cu") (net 28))
 (segment (start 109.11 156.135001) (end 109.11 155.79) (width 0.2) (layer "F.Cu") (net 28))
 (segment (start 109.01 159.09) (end 109.01 157.814999) (width 0.2) (layer "F.Cu") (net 28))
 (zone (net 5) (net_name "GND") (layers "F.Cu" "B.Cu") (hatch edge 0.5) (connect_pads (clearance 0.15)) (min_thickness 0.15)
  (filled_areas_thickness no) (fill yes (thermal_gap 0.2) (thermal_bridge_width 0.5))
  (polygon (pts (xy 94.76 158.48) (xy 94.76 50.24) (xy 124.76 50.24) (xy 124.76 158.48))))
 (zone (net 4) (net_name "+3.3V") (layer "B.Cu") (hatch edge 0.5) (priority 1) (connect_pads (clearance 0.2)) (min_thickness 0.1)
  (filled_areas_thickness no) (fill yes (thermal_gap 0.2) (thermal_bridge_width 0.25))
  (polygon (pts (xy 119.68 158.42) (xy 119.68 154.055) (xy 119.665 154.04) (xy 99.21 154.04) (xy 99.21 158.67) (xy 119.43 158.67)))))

